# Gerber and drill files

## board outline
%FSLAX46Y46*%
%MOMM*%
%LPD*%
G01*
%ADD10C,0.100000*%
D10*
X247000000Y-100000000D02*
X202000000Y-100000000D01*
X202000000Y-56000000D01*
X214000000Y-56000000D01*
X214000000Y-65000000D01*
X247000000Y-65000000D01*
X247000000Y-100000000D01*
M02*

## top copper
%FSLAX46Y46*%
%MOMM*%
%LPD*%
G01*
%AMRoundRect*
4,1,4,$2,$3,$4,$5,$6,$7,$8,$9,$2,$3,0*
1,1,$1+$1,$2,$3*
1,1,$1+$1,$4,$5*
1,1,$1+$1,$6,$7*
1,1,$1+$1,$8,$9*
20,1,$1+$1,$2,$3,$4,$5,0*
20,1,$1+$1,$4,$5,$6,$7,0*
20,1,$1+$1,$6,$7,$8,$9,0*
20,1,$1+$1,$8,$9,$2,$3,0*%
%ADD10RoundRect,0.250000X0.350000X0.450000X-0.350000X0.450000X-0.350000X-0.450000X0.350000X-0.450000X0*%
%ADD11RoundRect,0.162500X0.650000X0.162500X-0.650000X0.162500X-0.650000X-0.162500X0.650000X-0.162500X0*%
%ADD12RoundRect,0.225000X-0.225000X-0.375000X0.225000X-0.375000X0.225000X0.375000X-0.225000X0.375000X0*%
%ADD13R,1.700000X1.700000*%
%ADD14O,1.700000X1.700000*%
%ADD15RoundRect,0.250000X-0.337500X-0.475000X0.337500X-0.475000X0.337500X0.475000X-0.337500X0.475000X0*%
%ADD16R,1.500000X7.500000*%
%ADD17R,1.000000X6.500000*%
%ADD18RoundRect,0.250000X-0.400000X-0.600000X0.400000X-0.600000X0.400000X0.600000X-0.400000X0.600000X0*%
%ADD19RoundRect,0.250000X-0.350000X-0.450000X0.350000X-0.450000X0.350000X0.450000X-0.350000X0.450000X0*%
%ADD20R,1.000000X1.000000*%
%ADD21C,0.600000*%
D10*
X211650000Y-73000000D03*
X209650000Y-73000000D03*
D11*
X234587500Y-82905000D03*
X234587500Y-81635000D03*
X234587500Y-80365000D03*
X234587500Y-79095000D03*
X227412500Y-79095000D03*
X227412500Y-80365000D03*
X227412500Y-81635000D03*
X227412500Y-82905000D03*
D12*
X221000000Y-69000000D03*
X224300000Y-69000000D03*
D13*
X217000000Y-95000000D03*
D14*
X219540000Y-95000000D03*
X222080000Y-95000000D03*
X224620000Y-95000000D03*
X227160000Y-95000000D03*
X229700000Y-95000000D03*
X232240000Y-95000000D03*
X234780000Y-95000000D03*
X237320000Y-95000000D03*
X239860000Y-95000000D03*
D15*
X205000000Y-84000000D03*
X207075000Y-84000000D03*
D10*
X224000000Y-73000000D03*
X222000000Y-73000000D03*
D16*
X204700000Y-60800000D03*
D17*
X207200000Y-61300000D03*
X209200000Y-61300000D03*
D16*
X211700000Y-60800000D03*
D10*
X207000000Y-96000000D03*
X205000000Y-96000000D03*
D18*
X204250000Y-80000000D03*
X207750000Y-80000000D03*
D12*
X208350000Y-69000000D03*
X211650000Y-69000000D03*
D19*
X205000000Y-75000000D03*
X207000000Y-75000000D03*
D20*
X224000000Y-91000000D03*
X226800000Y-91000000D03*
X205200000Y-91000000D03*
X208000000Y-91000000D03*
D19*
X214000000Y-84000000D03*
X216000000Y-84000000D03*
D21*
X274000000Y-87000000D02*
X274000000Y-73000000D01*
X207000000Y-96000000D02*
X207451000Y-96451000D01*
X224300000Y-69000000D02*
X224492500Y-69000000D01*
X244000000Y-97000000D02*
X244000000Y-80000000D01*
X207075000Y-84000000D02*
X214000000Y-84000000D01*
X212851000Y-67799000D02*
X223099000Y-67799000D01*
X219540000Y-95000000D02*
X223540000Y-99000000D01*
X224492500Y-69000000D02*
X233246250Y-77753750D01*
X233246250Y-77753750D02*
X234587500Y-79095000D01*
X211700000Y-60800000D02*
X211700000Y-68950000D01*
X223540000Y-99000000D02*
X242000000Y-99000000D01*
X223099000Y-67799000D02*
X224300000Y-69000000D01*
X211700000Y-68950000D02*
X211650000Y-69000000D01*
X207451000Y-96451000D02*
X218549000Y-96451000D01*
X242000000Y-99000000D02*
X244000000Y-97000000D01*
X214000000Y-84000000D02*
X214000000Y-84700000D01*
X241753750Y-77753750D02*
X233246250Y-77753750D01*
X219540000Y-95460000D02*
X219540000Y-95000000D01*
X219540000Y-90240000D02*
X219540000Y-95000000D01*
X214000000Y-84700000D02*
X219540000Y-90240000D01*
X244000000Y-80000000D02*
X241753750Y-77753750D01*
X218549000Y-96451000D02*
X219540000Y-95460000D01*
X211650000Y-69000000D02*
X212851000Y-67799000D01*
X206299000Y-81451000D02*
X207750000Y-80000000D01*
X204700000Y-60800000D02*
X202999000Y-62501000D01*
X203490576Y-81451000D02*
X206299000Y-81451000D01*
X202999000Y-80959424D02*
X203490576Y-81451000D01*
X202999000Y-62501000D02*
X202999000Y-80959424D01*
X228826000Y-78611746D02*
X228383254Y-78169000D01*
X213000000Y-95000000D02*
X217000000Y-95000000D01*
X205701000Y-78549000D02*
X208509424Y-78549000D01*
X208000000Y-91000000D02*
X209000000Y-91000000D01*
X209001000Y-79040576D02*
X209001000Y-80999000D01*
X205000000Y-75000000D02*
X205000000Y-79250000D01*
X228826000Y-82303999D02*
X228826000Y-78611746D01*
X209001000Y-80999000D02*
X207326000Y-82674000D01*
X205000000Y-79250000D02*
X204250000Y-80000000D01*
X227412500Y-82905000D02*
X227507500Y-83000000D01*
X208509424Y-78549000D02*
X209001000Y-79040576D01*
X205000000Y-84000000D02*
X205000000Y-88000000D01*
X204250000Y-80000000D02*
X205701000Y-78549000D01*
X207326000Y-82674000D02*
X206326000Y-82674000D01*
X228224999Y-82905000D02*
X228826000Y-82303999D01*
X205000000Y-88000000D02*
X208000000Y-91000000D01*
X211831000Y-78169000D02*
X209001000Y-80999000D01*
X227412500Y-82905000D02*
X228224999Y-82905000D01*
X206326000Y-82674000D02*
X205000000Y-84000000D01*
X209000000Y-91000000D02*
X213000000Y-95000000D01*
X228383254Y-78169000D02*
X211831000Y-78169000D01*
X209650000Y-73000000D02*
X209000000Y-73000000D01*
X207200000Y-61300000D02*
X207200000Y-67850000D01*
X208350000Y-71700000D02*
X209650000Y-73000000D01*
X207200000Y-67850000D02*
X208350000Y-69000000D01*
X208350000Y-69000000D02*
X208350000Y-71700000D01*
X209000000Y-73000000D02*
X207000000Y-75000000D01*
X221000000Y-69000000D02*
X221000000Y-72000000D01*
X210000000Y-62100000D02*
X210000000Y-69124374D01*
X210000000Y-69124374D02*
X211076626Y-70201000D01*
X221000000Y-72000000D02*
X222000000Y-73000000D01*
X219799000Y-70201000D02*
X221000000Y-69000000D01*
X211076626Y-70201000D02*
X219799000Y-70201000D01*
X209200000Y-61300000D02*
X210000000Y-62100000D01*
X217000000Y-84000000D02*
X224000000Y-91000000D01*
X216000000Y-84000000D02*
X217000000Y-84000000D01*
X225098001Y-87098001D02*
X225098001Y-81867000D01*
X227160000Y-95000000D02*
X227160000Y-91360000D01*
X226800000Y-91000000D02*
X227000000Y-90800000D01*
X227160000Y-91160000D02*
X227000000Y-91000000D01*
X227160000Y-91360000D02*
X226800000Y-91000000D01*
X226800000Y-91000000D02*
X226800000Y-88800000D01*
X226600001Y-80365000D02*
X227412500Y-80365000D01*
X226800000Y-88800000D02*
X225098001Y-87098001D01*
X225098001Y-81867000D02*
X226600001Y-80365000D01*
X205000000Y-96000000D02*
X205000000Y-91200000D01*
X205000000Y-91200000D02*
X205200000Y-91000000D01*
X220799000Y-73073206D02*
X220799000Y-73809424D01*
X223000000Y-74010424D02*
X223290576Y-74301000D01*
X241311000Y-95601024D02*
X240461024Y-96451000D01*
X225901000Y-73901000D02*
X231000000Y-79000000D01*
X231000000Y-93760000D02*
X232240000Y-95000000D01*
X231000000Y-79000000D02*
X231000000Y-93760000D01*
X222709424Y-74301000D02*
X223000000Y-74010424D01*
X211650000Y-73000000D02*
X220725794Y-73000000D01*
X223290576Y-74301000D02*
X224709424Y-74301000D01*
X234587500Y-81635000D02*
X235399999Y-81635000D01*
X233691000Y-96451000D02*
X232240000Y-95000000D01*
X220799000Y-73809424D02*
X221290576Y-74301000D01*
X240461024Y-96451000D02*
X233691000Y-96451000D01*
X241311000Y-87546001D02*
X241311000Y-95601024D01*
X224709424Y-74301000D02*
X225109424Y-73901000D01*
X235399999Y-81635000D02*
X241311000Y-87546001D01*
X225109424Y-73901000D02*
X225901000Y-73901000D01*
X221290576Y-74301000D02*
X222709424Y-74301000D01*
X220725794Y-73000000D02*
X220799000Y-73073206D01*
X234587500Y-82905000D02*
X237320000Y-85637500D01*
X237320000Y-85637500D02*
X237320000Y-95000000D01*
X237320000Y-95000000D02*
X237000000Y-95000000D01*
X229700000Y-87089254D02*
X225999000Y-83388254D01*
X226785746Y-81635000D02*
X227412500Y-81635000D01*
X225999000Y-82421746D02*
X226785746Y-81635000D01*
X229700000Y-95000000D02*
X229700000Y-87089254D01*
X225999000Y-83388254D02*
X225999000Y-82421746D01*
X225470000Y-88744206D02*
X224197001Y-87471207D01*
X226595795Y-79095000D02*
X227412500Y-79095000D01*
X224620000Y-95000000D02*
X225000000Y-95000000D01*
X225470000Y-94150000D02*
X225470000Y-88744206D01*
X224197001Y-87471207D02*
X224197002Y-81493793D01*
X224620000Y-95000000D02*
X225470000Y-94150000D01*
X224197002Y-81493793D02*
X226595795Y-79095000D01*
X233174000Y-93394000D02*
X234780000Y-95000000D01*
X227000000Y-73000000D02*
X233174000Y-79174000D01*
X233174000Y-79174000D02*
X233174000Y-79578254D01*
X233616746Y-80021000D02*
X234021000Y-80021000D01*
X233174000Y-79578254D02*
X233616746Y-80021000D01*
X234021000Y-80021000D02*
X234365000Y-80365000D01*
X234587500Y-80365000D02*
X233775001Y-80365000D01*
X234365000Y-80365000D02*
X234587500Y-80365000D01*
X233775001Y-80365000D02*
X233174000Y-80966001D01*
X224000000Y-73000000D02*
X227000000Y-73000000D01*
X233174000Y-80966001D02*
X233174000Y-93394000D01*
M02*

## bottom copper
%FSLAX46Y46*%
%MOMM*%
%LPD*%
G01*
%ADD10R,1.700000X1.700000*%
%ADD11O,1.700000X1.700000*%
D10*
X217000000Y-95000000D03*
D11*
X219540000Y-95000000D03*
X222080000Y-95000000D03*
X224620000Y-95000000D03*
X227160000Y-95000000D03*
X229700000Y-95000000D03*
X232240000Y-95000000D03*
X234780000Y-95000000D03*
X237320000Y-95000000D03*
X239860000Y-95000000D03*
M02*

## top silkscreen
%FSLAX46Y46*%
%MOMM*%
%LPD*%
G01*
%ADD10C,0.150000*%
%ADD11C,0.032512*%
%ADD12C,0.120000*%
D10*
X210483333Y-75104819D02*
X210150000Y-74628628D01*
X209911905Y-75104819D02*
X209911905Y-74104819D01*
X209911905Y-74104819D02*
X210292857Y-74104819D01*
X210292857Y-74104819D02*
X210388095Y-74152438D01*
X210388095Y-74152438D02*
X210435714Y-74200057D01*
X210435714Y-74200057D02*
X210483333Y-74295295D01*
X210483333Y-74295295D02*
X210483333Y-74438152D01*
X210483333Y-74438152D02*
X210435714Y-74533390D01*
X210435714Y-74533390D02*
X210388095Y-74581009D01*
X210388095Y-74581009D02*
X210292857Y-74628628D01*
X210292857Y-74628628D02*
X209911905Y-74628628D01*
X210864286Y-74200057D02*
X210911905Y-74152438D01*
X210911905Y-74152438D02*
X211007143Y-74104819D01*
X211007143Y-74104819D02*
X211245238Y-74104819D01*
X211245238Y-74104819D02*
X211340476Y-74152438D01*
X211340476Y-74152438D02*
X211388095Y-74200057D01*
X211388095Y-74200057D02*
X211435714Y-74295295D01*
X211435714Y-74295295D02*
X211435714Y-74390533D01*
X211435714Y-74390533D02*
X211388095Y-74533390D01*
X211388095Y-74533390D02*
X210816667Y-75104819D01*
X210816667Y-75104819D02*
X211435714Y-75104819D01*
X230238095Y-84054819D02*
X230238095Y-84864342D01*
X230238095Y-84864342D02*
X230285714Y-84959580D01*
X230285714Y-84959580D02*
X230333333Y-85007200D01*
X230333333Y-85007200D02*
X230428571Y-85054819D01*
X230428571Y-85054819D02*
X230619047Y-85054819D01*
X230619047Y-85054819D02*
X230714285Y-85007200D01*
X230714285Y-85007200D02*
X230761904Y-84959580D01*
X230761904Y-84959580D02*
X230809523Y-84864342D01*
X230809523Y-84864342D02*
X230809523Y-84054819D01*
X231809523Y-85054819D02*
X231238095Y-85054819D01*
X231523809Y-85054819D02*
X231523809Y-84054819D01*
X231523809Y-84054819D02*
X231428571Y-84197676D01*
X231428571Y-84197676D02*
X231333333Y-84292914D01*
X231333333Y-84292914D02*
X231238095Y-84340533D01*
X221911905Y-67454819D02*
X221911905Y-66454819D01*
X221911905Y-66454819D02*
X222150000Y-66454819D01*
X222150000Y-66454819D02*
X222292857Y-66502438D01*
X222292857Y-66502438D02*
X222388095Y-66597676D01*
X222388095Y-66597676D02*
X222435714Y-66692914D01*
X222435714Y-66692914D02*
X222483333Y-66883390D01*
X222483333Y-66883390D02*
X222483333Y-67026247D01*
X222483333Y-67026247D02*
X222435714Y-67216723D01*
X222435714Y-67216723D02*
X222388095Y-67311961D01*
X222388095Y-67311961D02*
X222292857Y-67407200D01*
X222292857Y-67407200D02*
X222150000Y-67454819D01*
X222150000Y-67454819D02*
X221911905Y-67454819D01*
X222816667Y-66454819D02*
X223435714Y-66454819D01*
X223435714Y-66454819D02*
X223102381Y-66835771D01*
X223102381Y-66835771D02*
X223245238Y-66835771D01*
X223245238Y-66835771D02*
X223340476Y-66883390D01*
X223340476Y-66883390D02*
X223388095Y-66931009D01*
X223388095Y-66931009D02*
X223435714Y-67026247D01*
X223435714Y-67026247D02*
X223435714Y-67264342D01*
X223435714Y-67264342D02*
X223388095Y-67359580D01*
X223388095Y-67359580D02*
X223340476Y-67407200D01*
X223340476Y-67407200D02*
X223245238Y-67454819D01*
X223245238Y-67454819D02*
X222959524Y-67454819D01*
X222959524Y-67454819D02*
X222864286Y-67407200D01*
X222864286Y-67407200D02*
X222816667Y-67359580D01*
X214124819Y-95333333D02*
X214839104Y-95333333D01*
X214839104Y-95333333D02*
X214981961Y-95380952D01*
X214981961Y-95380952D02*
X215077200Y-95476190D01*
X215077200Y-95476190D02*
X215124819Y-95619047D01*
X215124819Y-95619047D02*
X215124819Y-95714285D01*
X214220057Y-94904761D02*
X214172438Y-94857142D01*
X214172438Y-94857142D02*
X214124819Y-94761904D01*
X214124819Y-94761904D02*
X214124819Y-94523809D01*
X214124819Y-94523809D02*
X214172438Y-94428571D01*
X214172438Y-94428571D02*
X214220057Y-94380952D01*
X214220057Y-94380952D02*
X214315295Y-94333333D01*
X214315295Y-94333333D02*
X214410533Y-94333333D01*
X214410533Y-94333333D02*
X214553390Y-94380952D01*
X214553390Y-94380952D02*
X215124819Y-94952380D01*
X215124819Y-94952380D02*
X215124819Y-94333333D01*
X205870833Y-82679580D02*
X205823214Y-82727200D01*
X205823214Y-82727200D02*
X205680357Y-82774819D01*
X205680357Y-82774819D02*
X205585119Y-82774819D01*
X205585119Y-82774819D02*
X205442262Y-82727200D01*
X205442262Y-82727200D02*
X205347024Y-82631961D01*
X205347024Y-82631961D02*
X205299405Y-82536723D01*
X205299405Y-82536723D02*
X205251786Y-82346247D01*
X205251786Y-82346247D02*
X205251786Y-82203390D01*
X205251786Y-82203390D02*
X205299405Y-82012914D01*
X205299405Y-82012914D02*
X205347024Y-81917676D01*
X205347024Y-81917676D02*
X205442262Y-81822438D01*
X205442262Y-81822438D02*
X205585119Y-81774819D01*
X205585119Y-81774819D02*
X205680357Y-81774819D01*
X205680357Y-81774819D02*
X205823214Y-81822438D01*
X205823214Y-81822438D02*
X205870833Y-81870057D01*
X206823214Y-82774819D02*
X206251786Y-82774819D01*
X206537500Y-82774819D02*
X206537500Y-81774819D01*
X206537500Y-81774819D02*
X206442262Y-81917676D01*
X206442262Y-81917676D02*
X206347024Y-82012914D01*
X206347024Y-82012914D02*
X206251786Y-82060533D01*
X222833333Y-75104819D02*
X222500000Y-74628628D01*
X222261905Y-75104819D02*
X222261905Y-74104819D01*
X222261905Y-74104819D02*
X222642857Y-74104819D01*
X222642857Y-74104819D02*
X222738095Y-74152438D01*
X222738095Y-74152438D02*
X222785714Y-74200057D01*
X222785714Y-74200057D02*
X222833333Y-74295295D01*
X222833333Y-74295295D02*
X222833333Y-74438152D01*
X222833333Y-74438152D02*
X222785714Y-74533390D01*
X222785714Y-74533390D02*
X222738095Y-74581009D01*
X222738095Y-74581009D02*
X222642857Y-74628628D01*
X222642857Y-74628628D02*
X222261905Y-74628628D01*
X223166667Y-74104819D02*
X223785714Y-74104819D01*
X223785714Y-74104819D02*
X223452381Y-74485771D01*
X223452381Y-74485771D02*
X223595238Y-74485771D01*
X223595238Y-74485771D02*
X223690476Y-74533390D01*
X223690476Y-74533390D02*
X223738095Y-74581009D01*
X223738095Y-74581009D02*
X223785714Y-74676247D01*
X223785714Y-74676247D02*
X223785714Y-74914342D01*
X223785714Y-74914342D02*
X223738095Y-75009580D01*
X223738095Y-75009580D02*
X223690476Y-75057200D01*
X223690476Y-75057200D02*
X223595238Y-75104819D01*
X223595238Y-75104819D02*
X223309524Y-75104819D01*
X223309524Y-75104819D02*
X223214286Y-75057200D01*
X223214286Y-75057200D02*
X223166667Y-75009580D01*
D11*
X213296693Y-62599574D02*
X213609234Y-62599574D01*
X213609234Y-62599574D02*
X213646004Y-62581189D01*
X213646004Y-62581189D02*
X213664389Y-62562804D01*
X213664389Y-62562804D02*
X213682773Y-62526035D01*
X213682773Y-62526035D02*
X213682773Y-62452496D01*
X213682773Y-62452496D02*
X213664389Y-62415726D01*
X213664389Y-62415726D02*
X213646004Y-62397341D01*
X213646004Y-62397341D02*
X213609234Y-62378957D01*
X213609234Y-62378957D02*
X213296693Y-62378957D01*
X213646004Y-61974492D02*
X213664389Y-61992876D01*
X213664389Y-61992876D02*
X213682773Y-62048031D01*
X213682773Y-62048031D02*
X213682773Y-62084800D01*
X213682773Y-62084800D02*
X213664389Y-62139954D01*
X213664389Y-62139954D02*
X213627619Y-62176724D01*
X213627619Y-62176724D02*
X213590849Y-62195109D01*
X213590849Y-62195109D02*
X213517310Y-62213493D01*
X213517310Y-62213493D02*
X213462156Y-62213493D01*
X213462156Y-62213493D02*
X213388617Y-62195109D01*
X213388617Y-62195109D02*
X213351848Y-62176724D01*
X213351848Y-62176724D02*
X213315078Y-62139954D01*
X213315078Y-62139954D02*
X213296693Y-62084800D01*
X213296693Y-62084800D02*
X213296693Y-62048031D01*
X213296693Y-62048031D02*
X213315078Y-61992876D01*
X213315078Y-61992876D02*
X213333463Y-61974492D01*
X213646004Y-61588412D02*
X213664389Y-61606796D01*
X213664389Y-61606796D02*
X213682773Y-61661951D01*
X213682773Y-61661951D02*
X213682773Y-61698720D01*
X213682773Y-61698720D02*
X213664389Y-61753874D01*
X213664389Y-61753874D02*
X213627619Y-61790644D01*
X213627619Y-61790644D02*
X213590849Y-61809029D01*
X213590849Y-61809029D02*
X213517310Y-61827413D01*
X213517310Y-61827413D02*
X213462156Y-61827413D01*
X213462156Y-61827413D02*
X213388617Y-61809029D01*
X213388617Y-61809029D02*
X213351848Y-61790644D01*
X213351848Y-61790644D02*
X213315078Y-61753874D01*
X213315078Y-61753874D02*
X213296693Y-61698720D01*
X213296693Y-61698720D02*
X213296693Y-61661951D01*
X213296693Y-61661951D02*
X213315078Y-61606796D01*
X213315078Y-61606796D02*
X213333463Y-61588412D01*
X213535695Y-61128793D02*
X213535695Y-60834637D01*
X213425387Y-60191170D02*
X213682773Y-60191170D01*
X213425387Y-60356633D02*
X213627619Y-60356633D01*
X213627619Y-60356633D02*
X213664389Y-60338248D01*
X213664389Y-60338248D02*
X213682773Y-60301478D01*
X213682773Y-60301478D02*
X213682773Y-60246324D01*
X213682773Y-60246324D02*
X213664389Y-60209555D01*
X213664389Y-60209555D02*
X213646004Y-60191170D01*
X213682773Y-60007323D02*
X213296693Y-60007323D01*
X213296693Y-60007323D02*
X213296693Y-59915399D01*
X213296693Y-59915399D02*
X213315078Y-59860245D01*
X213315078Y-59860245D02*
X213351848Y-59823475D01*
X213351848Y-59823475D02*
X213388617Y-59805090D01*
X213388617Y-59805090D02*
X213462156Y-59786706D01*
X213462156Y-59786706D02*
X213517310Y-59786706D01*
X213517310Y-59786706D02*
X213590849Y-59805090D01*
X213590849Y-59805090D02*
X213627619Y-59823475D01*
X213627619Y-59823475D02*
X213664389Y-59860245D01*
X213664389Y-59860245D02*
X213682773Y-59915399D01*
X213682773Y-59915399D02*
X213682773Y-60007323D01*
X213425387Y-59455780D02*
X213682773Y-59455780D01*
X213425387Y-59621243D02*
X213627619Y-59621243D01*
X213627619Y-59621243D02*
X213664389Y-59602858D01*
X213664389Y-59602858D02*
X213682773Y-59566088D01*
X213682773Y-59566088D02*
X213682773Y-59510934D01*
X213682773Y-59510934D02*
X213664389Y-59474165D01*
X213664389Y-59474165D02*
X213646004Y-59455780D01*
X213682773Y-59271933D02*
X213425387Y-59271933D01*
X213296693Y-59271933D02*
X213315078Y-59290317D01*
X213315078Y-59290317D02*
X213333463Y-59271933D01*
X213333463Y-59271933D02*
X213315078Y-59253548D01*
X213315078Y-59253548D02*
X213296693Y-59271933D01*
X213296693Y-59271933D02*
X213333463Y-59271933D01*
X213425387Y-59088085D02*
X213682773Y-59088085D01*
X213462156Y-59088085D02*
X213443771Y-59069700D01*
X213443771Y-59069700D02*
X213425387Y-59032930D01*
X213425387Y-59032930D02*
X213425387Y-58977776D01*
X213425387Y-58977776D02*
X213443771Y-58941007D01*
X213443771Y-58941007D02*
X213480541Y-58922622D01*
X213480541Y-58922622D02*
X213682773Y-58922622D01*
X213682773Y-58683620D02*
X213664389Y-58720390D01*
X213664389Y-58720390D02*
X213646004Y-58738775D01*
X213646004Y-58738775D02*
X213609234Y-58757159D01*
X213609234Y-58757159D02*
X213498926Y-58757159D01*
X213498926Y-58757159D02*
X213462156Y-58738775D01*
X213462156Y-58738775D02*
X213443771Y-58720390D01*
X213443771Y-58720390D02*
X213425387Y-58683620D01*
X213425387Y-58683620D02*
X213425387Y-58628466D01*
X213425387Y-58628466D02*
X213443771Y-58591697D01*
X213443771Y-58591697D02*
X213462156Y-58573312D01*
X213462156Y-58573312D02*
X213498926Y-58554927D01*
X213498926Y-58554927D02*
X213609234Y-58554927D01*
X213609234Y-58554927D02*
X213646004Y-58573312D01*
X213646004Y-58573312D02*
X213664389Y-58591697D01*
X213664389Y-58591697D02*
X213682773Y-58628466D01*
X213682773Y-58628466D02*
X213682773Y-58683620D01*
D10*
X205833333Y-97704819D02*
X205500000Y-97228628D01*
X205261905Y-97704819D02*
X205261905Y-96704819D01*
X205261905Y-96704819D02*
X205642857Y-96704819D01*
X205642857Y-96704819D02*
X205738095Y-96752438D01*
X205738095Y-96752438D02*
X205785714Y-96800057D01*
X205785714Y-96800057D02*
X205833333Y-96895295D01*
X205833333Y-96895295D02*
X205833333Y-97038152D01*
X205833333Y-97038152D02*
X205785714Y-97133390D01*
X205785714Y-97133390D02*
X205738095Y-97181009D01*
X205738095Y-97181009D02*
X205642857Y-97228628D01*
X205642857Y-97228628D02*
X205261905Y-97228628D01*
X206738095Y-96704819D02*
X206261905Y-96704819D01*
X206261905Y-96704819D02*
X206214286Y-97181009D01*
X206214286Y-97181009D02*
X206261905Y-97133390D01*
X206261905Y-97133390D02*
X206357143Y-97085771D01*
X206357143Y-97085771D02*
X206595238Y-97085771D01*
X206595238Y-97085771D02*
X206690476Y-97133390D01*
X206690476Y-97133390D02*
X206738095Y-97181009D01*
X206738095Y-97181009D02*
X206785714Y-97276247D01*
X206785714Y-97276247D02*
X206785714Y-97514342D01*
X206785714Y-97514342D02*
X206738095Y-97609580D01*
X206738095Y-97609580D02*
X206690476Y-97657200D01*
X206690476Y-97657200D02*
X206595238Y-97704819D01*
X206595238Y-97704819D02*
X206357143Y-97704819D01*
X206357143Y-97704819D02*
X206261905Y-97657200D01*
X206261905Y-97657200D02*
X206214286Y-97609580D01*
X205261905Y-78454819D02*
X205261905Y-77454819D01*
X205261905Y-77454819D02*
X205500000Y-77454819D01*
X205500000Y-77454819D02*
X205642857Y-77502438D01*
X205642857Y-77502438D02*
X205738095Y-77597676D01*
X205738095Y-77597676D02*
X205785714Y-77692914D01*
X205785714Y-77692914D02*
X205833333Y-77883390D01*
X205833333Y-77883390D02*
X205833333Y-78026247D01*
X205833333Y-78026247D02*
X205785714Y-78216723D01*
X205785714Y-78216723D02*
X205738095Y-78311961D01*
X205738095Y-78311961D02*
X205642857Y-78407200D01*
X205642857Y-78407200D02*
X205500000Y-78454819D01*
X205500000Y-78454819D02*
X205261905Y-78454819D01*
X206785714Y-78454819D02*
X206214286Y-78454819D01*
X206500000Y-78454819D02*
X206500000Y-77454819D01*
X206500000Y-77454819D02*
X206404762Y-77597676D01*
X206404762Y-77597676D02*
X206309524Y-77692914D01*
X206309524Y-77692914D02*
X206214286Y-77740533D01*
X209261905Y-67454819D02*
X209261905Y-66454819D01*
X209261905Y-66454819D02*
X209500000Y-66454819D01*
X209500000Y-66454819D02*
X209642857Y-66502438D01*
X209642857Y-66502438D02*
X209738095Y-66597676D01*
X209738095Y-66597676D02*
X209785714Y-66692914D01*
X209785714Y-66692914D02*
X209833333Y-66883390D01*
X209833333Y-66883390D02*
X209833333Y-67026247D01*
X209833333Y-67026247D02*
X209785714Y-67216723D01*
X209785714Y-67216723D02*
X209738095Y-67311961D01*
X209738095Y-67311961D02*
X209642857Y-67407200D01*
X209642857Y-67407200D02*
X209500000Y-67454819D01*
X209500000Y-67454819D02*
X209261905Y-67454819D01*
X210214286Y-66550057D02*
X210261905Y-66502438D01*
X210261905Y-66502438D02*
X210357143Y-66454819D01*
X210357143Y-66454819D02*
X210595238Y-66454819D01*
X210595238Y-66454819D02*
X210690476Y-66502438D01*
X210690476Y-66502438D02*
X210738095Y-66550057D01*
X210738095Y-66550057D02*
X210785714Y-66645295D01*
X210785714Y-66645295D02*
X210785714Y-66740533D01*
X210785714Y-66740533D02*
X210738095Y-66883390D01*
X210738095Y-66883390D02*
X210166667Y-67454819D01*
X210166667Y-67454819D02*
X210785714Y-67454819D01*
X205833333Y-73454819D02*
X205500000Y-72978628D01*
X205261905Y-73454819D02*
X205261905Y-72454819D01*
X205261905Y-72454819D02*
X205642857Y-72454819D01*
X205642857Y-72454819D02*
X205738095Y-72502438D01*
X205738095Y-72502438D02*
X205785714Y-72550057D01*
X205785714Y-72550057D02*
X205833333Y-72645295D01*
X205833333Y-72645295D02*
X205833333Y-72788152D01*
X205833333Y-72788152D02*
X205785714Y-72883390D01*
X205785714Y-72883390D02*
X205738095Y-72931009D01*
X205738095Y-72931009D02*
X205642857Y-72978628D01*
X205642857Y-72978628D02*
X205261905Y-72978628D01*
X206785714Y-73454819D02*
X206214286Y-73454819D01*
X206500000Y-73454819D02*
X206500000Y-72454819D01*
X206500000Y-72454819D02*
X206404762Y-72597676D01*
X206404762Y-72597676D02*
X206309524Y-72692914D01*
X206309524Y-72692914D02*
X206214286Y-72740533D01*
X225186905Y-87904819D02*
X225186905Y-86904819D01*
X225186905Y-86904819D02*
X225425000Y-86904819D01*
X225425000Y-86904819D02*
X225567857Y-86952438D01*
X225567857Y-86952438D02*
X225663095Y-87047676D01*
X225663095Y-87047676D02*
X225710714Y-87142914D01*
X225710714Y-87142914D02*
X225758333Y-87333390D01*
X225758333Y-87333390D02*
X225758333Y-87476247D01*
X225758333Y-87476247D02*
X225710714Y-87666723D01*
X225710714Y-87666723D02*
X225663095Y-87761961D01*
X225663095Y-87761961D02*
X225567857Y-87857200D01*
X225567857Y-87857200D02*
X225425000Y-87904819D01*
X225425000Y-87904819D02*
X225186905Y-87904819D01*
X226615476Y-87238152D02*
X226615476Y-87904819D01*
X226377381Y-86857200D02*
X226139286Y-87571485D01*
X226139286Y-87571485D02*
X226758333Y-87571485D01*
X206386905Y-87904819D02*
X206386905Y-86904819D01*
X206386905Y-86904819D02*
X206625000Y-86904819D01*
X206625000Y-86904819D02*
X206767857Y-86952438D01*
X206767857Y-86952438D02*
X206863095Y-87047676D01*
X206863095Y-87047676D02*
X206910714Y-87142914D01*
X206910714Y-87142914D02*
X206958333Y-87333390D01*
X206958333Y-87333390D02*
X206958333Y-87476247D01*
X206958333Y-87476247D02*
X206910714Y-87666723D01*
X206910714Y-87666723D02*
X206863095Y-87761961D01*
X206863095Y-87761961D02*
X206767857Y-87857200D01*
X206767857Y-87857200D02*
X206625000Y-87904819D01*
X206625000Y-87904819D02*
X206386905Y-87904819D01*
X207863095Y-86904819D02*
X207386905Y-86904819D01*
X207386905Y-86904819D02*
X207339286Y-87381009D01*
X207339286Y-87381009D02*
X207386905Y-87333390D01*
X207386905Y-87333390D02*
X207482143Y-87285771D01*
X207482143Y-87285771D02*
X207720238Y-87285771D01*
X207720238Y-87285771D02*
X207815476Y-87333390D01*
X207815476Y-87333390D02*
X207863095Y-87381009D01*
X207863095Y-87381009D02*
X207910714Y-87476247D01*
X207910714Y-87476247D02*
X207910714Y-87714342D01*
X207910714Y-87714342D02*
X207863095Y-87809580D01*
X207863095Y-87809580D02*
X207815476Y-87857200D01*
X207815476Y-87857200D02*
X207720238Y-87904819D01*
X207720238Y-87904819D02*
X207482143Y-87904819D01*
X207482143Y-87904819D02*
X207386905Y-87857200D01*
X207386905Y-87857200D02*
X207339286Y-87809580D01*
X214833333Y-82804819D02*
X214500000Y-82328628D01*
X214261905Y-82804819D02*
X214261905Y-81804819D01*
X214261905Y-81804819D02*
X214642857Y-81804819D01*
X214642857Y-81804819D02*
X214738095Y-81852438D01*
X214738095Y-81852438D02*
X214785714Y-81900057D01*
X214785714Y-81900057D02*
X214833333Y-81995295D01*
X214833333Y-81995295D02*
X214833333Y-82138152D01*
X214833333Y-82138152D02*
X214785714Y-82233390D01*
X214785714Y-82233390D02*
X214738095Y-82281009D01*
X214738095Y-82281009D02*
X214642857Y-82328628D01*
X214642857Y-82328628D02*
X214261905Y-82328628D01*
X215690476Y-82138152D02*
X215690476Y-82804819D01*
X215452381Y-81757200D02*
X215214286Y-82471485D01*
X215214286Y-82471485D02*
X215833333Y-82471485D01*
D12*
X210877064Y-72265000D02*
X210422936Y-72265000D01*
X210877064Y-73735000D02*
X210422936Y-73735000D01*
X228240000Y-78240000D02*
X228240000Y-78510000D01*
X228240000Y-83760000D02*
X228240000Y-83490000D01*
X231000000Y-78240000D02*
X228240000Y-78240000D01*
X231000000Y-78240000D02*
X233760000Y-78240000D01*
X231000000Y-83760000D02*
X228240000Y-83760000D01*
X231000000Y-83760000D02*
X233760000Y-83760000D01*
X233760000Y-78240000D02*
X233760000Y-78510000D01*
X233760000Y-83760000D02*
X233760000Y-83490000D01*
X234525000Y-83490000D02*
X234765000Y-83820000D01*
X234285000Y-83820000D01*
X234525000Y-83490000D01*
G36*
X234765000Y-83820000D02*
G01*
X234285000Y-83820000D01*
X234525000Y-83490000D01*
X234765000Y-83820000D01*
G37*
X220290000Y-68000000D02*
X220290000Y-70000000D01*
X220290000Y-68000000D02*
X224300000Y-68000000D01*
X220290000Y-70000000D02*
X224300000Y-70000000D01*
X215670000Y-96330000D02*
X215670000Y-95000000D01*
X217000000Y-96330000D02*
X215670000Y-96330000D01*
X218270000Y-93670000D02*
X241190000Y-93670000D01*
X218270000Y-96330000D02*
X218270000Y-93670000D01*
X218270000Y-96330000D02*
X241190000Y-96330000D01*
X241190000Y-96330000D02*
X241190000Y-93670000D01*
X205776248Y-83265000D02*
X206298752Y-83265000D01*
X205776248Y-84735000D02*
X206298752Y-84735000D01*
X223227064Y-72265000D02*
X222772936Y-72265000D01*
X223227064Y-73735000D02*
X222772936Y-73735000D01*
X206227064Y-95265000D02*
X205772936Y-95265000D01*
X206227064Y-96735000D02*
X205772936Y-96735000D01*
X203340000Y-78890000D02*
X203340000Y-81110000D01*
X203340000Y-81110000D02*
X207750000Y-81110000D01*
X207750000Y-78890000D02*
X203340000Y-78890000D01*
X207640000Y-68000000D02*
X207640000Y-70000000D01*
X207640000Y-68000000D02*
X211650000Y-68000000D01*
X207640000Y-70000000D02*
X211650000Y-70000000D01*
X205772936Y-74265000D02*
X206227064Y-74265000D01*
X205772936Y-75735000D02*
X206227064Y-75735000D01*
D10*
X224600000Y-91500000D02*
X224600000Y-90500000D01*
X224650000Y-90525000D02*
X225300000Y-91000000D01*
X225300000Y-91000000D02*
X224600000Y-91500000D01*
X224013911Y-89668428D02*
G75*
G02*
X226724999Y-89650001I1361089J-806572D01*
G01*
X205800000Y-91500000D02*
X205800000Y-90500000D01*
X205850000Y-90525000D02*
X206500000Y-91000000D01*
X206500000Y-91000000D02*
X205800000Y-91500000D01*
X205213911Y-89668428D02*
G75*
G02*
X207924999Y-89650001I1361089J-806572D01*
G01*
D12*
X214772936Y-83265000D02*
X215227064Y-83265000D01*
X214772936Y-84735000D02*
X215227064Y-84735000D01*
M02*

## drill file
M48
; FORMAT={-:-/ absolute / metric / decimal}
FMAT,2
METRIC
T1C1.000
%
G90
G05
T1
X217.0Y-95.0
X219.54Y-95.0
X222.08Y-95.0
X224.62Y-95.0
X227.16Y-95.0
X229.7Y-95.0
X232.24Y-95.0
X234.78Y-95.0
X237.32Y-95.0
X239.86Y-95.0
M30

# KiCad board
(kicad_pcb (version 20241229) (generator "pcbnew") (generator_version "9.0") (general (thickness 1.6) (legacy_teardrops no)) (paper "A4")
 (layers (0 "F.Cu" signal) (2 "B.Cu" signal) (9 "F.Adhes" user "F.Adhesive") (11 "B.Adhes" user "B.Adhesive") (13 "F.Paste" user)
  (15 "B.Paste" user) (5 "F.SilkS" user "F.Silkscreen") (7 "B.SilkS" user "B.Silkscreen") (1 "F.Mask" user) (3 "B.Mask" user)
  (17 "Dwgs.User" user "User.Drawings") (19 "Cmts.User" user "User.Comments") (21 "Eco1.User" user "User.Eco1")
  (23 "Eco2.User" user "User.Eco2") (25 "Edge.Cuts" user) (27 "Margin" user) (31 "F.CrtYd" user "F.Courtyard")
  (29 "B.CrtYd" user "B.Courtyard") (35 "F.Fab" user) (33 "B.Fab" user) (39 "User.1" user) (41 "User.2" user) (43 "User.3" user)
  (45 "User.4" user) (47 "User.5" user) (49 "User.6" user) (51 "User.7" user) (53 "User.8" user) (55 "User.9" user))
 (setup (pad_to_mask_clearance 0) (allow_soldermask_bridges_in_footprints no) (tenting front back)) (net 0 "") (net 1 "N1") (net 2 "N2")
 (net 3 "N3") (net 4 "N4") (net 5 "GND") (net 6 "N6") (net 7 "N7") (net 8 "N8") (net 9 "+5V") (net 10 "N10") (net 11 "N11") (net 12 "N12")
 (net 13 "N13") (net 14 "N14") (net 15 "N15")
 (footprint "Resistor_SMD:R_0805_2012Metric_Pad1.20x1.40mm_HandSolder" (layer "F.Cu") (at 210.65 73 180)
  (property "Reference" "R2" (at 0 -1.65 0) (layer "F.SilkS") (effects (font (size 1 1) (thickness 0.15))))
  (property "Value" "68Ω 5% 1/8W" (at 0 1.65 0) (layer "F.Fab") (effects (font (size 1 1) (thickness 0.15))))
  (fp_line (start -0.227064 0.735) (end 0.227064 0.735) (stroke (width 0.12) (type solid)) (layer "F.SilkS"))
  (fp_line (start -0.227064 -0.735) (end 0.227064 -0.735) (stroke (width 0.12) (type solid)) (layer "F.SilkS"))
  (pad "1" smd roundrect (at -1 0 180) (size 1.2 1.4) (layers "F.Cu" "F.Mask" "F.Paste") (roundrect_rratio 0.208333) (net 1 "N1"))
  (pad "2" smd roundrect (at 1 0 180) (size 1.2 1.4) (layers "F.Cu" "F.Mask" "F.Paste") (roundrect_rratio 0.208333) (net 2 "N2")))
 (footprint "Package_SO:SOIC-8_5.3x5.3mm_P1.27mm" (layer "F.Cu") (at 231 81 180)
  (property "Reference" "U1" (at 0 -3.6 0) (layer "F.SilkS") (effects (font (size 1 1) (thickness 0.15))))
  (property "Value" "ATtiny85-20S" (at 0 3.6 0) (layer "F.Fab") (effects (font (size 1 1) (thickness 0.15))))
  (fp_line (start 2.76 2.76) (end 2.76 2.49) (stroke (width 0.12) (type solid)) (layer "F.SilkS"))
  (fp_line (start 2.76 -2.76) (end 2.76 -2.49) (stroke (width 0.12) (type solid)) (layer "F.SilkS"))
  (fp_line (start 0 2.76) (end 2.76 2.76) (stroke (width 0.12) (type solid)) (layer "F.SilkS"))
  (fp_line (start 0 2.76) (end -2.76 2.76) (stroke (width 0.12) (type solid)) (layer "F.SilkS"))
  (fp_line (start 0 -2.76) (end 2.76 -2.76) (stroke (width 0.12) (type solid)) (layer "F.SilkS"))
  (fp_line (start 0 -2.76) (end -2.76 -2.76) (stroke (width 0.12) (type solid)) (layer "F.SilkS"))
  (fp_line (start -2.76 2.76) (end -2.76 2.49) (stroke (width 0.12) (type solid)) (layer "F.SilkS"))
  (fp_line (start -2.76 -2.76) (end -2.76 -2.49) (stroke (width 0.12) (type solid)) (layer "F.SilkS"))
  (fp_poly
   (pts (xy -3.525 -2.49) (xy -3.765 -2.82) (xy -3.285 -2.82) (xy -3.525 -2.49)) (stroke (width 0.12) (type solid)) (fill yes)
   (layer "F.SilkS"))
  (pad "1" smd roundrect (at -3.5875 -1.905 180) (size 1.625 0.65) (layers "F.Cu" "F.Mask" "F.Paste") (roundrect_rratio 0.25) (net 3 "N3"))
  (pad "2" smd roundrect (at -3.5875 -0.635 180) (size 1.625 0.65) (layers "F.Cu" "F.Mask" "F.Paste") (roundrect_rratio 0.25) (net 1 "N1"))
  (pad "3" smd roundrect (at -3.5875 0.635 180) (size 1.625 0.65) (layers "F.Cu" "F.Mask" "F.Paste") (roundrect_rratio 0.25) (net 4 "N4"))
  (pad "4" smd roundrect (at -3.5875 1.905 180) (size 1.625 0.65) (layers "F.Cu" "F.Mask" "F.Paste") (roundrect_rratio 0.25) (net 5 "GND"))
  (pad "5" smd roundrect (at 3.5875 1.905 180) (size 1.625 0.65) (layers "F.Cu" "F.Mask" "F.Paste") (roundrect_rratio 0.25) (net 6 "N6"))
  (pad "6" smd roundrect (at 3.5875 0.635 180) (size 1.625 0.65) (layers "F.Cu" "F.Mask" "F.Paste") (roundrect_rratio 0.25) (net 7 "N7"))
  (pad "7" smd roundrect (at 3.5875 -0.635 180) (size 1.625 0.65) (layers "F.Cu" "F.Mask" "F.Paste") (roundrect_rratio 0.25) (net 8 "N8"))
  (pad "8" smd roundrect (at 3.5875 -1.905 180) (size 1.625 0.65) (layers "F.Cu" "F.Mask" "F.Paste") (roundrect_rratio 0.25) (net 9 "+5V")))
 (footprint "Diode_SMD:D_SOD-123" (layer "F.Cu") (at 222.65 69)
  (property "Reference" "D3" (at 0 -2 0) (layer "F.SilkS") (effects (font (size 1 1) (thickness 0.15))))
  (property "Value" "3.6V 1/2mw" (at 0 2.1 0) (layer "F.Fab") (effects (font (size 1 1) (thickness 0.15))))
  (fp_line (start -2.36 -1) (end -2.36 1) (stroke (width 0.12) (type solid)) (layer "F.SilkS"))
  (fp_line (start -2.36 -1) (end 1.65 -1) (stroke (width 0.12) (type solid)) (layer "F.SilkS"))
  (fp_line (start -2.36 1) (end 1.65 1) (stroke (width 0.12) (type solid)) (layer "F.SilkS"))
  (pad "1" smd roundrect (at -1.65 0) (size 0.9 1.2) (layers "F.Cu" "F.Mask" "F.Paste") (roundrect_rratio 0.25) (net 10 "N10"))
  (pad "2" smd roundrect (at 1.65 0) (size 0.9 1.2) (layers "F.Cu" "F.Mask" "F.Paste") (roundrect_rratio 0.25) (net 5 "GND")))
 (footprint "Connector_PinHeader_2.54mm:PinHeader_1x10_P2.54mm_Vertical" (layer "F.Cu") (at 217 95 90)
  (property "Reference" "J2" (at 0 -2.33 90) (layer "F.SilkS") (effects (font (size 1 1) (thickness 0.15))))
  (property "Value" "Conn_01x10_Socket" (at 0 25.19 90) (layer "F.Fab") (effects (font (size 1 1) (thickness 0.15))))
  (fp_line (start -1.33 -1.33) (end 0 -1.33) (stroke (width 0.12) (type solid)) (layer "F.SilkS"))
  (fp_line (start -1.33 0) (end -1.33 -1.33) (stroke (width 0.12) (type solid)) (layer "F.SilkS"))
  (fp_line (start 1.33 1.27) (end 1.33 24.19) (stroke (width 0.12) (type solid)) (layer "F.SilkS"))
  (fp_line (start -1.33 1.27) (end 1.33 1.27) (stroke (width 0.12) (type solid)) (layer "F.SilkS"))
  (fp_line (start -1.33 1.27) (end -1.33 24.19) (stroke (width 0.12) (type solid)) (layer "F.SilkS"))
  (fp_line (start -1.33 24.19) (end 1.33 24.19) (stroke (width 0.12) (type solid)) (layer "F.SilkS"))
  (pad "1" thru_hole rect (at 0 0 90) (size 1.7 1.7) (drill 1) (layers "*.Cu" "*.Mask") (remove_unused_layers no) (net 9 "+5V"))
  (pad "2" thru_hole oval (at 0 2.54 90) (size 1.7 1.7) (drill 1) (layers "*.Cu" "*.Mask") (remove_unused_layers no) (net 5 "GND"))
  (pad "3" thru_hole oval (at 0 5.08 90) (size 1.7 1.7) (drill 1) (layers "*.Cu" "*.Mask") (remove_unused_layers no) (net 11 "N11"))
  (pad "4" thru_hole oval (at 0 7.62 90) (size 1.7 1.7) (drill 1) (layers "*.Cu" "*.Mask") (remove_unused_layers no) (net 6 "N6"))
  (pad "5" thru_hole oval (at 0 10.16 90) (size 1.7 1.7) (drill 1) (layers "*.Cu" "*.Mask") (remove_unused_layers no) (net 7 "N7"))
  (pad "6" thru_hole oval (at 0 12.7 90) (size 1.7 1.7) (drill 1) (layers "*.Cu" "*.Mask") (remove_unused_layers no) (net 8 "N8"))
  (pad "7" thru_hole oval (at 0 15.24 90) (size 1.7 1.7) (drill 1) (layers "*.Cu" "*.Mask") (remove_unused_layers no) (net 1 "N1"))
  (pad "8" thru_hole oval (at 0 17.78 90) (size 1.7 1.7) (drill 1) (layers "*.Cu" "*.Mask") (remove_unused_layers no) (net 4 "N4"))
  (pad "9" thru_hole oval (at 0 20.32 90) (size 1.7 1.7) (drill 1) (layers "*.Cu" "*.Mask") (remove_unused_layers no) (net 3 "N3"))
  (pad "10" thru_hole oval (at 0 22.86 90) (size 1.7 1.7) (drill 1) (layers "*.Cu" "*.Mask") (remove_unused_layers no) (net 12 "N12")))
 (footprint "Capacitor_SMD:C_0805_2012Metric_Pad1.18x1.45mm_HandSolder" (layer "F.Cu") (at 206.0375 84)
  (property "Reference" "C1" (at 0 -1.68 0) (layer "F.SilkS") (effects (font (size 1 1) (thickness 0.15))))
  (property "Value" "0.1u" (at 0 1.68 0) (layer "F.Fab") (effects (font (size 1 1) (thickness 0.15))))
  (fp_line (start -0.261252 -0.735) (end 0.261252 -0.735) (stroke (width 0.12) (type solid)) (layer "F.SilkS"))
  (fp_line (start -0.261252 0.735) (end 0.261252 0.735) (stroke (width 0.12) (type solid)) (layer "F.SilkS"))
  (pad "1" smd roundrect (at -1.0375 0) (size 1.175 1.45) (layers "F.Cu" "F.Mask" "F.Paste") (roundrect_rratio 0.212766) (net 9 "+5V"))
  (pad "2" smd roundrect (at 1.0375 0) (size 1.175 1.45) (layers "F.Cu" "F.Mask" "F.Paste") (roundrect_rratio 0.212766) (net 5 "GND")))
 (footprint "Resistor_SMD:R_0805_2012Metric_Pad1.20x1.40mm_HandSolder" (layer "F.Cu") (at 223 73 180)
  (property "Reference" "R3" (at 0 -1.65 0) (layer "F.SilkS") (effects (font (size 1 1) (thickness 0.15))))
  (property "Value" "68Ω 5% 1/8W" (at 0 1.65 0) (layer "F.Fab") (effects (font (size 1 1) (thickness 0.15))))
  (fp_line (start -0.227064 0.735) (end 0.227064 0.735) (stroke (width 0.12) (type solid)) (layer "F.SilkS"))
  (fp_line (start -0.227064 -0.735) (end 0.227064 -0.735) (stroke (width 0.12) (type solid)) (layer "F.SilkS"))
  (pad "1" smd roundrect (at -1 0 180) (size 1.2 1.4) (layers "F.Cu" "F.Mask" "F.Paste") (roundrect_rratio 0.208333) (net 4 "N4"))
  (pad "2" smd roundrect (at 1 0 180) (size 1.2 1.4) (layers "F.Cu" "F.Mask" "F.Paste") (roundrect_rratio 0.208333) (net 10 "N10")))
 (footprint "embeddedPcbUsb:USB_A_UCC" (layer "F.Cu") (at 208.2 61 -90)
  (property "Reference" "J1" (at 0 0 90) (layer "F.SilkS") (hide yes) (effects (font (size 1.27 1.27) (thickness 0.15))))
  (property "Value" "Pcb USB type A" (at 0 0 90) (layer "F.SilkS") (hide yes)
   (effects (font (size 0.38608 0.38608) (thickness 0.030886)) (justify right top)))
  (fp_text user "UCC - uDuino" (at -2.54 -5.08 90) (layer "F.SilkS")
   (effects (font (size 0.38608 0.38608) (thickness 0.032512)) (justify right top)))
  (pad "1" smd rect (at -0.2 3.5 270) (size 7.5 1.5) (layers "F.Cu" "F.Mask" "F.Paste") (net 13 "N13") (solder_mask_margin 0.1016))
  (pad "2" smd rect (at 0.3 1 270) (size 6.5 1) (layers "F.Cu" "F.Mask" "F.Paste") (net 2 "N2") (solder_mask_margin 0.1016))
  (pad "3" smd rect (at 0.3 -1 270) (size 6.5 1) (layers "F.Cu" "F.Mask" "F.Paste") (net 10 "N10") (solder_mask_margin 0.1016))
  (pad "4" smd rect (at -0.2 -3.5 270) (size 7.5 1.5) (layers "F.Cu" "F.Mask" "F.Paste") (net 5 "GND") (solder_mask_margin 0.1016)))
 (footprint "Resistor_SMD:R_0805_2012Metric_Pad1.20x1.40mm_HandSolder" (layer "F.Cu") (at 206 96 180)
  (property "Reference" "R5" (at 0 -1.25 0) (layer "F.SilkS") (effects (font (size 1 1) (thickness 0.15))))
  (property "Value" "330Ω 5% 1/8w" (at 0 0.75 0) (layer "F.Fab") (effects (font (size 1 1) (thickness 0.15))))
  (fp_line (start -0.227064 0.735) (end 0.227064 0.735) (stroke (width 0.12) (type solid)) (layer "F.SilkS"))
  (fp_line (start -0.227064 -0.735) (end 0.227064 -0.735) (stroke (width 0.12) (type solid)) (layer "F.SilkS"))
  (pad "1" smd roundrect (at -1 0 180) (size 1.2 1.4) (layers "F.Cu" "F.Mask" "F.Paste") (roundrect_rratio 0.208333) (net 5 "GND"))
  (pad "2" smd roundrect (at 1 0 180) (size 1.2 1.4) (layers "F.Cu" "F.Mask" "F.Paste") (roundrect_rratio 0.208333) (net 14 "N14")))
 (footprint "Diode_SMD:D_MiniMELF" (layer "F.Cu") (at 206 80)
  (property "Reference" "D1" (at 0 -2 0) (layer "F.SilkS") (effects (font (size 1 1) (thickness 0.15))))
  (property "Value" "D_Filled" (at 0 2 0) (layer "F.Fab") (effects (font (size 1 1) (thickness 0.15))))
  (fp_line (start -2.66 -1.11) (end -2.66 1.11) (stroke (width 0.12) (type solid)) (layer "F.SilkS"))
  (fp_line (start -2.66 1.11) (end 1.75 1.11) (stroke (width 0.12) (type solid)) (layer "F.SilkS"))
  (fp_line (start 1.75 -1.11) (end -2.66 -1.11) (stroke (width 0.12) (type solid)) (layer "F.SilkS"))
  (pad "1" smd roundrect (at -1.75 0) (size 1.3 1.7) (layers "F.Cu" "F.Mask" "F.Paste") (roundrect_rratio 0.1923076923) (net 9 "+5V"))
  (pad "2" smd roundrect (at 1.75 0) (size 1.3 1.7) (layers "F.Cu" "F.Mask" "F.Paste") (roundrect_rratio 0.1923076923) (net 13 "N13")))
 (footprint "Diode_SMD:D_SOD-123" (layer "F.Cu") (at 210 69)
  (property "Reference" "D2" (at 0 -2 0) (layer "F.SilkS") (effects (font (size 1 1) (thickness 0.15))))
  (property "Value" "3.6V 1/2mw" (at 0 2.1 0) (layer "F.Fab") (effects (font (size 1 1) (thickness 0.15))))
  (fp_line (start -2.36 -1) (end -2.36 1) (stroke (width 0.12) (type solid)) (layer "F.SilkS"))
  (fp_line (start -2.36 -1) (end 1.65 -1) (stroke (width 0.12) (type solid)) (layer "F.SilkS"))
  (fp_line (start -2.36 1) (end 1.65 1) (stroke (width 0.12) (type solid)) (layer "F.SilkS"))
  (pad "1" smd roundrect (at -1.65 0) (size 0.9 1.2) (layers "F.Cu" "F.Mask" "F.Paste") (roundrect_rratio 0.25) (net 2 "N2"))
  (pad "2" smd roundrect (at 1.65 0) (size 0.9 1.2) (layers "F.Cu" "F.Mask" "F.Paste") (roundrect_rratio 0.25) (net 5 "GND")))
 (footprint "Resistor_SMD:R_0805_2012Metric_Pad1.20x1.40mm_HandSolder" (layer "F.Cu") (at 206 75)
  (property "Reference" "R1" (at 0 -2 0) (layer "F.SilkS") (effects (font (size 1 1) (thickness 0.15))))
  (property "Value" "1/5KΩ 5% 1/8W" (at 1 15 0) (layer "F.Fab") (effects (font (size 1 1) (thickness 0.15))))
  (fp_line (start -0.227064 -0.735) (end 0.227064 -0.735) (stroke (width 0.12) (type solid)) (layer "F.SilkS"))
  (fp_line (start -0.227064 0.735) (end 0.227064 0.735) (stroke (width 0.12) (type solid)) (layer "F.SilkS"))
  (pad "1" smd roundrect (at -1 0) (size 1.2 1.4) (layers "F.Cu" "F.Mask" "F.Paste") (roundrect_rratio 0.208333) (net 9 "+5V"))
  (pad "2" smd roundrect (at 1 0) (size 1.2 1.4) (layers "F.Cu" "F.Mask" "F.Paste") (roundrect_rratio 0.208333) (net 2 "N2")))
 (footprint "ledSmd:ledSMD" (layer "F.Cu") (at 225.8 91)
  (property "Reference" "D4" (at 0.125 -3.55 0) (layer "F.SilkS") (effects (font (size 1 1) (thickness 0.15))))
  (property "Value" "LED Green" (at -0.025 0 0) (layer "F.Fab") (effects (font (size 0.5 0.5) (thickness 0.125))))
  (fp_line (start -1.2 0.5) (end -1.2 -0.5) (stroke (width 0.15) (type solid)) (layer "F.SilkS"))
  (fp_line (start -1.15 -0.475) (end -0.5 0) (stroke (width 0.15) (type solid)) (layer "F.SilkS"))
  (fp_line (start -0.5 0) (end -1.2 0.5) (stroke (width 0.15) (type solid)) (layer "F.SilkS"))
  (fp_arc (start -1.786089 -1.331572) (mid -0.435753 -2.107089) (end 0.924999 -1.349999) (stroke (width 0.15) (type solid))
   (layer "F.SilkS"))
  (pad "1" smd rect (at -1.8 0) (size 1 1) (layers "F.Cu" "F.Mask" "F.Paste") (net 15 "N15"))
  (pad "2" smd rect (at 1 0) (size 1 1) (layers "F.Cu" "F.Mask" "F.Paste") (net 7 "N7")))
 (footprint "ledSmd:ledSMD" (layer "F.Cu") (at 207 91)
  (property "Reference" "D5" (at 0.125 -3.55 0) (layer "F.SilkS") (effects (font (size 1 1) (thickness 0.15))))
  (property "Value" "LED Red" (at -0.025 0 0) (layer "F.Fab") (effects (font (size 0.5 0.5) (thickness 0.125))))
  (fp_line (start -1.2 0.5) (end -1.2 -0.5) (stroke (width 0.15) (type solid)) (layer "F.SilkS"))
  (fp_line (start -1.15 -0.475) (end -0.5 0) (stroke (width 0.15) (type solid)) (layer "F.SilkS"))
  (fp_line (start -0.5 0) (end -1.2 0.5) (stroke (width 0.15) (type solid)) (layer "F.SilkS"))
  (fp_arc (start -1.786089 -1.331572) (mid -0.435753 -2.107089) (end 0.924999 -1.349999) (stroke (width 0.15) (type solid))
   (layer "F.SilkS"))
  (pad "1" smd rect (at -1.8 0) (size 1 1) (layers "F.Cu" "F.Mask" "F.Paste") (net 14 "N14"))
  (pad "2" smd rect (at 1 0) (size 1 1) (layers "F.Cu" "F.Mask" "F.Paste") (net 9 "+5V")))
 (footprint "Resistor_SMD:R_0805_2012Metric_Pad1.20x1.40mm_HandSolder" (layer "F.Cu") (at 215 84)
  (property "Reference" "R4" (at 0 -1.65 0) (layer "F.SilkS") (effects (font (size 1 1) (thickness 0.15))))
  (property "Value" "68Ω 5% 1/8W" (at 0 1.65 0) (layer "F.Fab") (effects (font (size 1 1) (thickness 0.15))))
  (fp_line (start -0.227064 -0.735) (end 0.227064 -0.735) (stroke (width 0.12) (type solid)) (layer "F.SilkS"))
  (fp_line (start -0.227064 0.735) (end 0.227064 0.735) (stroke (width 0.12) (type solid)) (layer "F.SilkS"))
  (pad "1" smd roundrect (at -1 0) (size 1.2 1.4) (layers "F.Cu" "F.Mask" "F.Paste") (roundrect_rratio 0.208333) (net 5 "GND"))
  (pad "2" smd roundrect (at 1 0) (size 1.2 1.4) (layers "F.Cu" "F.Mask" "F.Paste") (roundrect_rratio 0.208333) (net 15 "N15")))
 (gr_poly
  (pts (xy 247 100) (xy 202 100) (xy 202 56) (xy 214 56) (xy 214 65) (xy 247 65)) (stroke (width 0.1) (type solid)) (fill no)
  (layer "Edge.Cuts"))
 (segment (start 274 87) (end 274 73) (width 0.6) (layer "F.Cu") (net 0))
 (segment (start 207 96) (end 207.451 96.451) (width 0.6) (layer "F.Cu") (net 5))
 (segment (start 224.3 69) (end 224.4925 69) (width 0.6) (layer "F.Cu") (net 5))
 (segment (start 244 97) (end 244 80) (width 0.6) (layer "F.Cu") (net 5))
 (segment (start 207.075 84) (end 214 84) (width 0.6) (layer "F.Cu") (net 5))
 (segment (start 212.851 67.799) (end 223.099 67.799) (width 0.6) (layer "F.Cu") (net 5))
 (segment (start 219.54 95) (end 223.54 99) (width 0.6) (layer "F.Cu") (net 5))
 (segment (start 224.4925 69) (end 233.24625 77.75375) (width 0.6) (layer "F.Cu") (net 5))
 (segment (start 233.24625 77.75375) (end 234.5875 79.095) (width 0.6) (layer "F.Cu") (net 5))
 (segment (start 211.7 60.8) (end 211.7 68.95) (width 0.6) (layer "F.Cu") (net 5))
 (segment (start 223.54 99) (end 242 99) (width 0.6) (layer "F.Cu") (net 5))
 (segment (start 223.099 67.799) (end 224.3 69) (width 0.6) (layer "F.Cu") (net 5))
 (segment (start 211.7 68.95) (end 211.65 69) (width 0.6) (layer "F.Cu") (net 5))
 (segment (start 207.451 96.451) (end 218.549 96.451) (width 0.6) (layer "F.Cu") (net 5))
 (segment (start 242 99) (end 244 97) (width 0.6) (layer "F.Cu") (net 5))
 (segment (start 214 84) (end 214 84.7) (width 0.6) (layer "F.Cu") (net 5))
 (segment (start 241.75375 77.75375) (end 233.24625 77.75375) (width 0.6) (layer "F.Cu") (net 5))
 (segment (start 219.54 95.46) (end 219.54 95) (width 0.6) (layer "F.Cu") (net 5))
 (segment (start 219.54 90.24) (end 219.54 95) (width 0.6) (layer "F.Cu") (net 5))
 (segment (start 214 84.7) (end 219.54 90.24) (width 0.6) (layer "F.Cu") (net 5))
 (segment (start 244 80) (end 241.75375 77.75375) (width 0.6) (layer "F.Cu") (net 5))
 (segment (start 218.549 96.451) (end 219.54 95.46) (width 0.6) (layer "F.Cu") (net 5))
 (segment (start 211.65 69) (end 212.851 67.799) (width 0.6) (layer "F.Cu") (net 5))
 (segment (start 206.299 81.451) (end 207.75 80) (width 0.6) (layer "F.Cu") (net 13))
 (segment (start 204.7 60.8) (end 202.999 62.501) (width 0.6) (layer "F.Cu") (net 13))
 (segment (start 203.490576 81.451) (end 206.299 81.451) (width 0.6) (layer "F.Cu") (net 13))
 (segment (start 202.999 80.959424) (end 203.490576 81.451) (width 0.6) (layer "F.Cu") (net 13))
 (segment (start 202.999 62.501) (end 202.999 80.959424) (width 0.6) (layer "F.Cu") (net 13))
 (segment (start 228.826 78.611746) (end 228.383254 78.169) (width 0.6) (layer "F.Cu") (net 9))
 (segment (start 213 95) (end 217 95) (width 0.6) (layer "F.Cu") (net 9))
 (segment (start 205.701 78.549) (end 208.509424 78.549) (width 0.6) (layer "F.Cu") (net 9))
 (segment (start 208 91) (end 209 91) (width 0.6) (layer "F.Cu") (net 9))
 (segment (start 209.001 79.040576) (end 209.001 80.999) (width 0.6) (layer "F.Cu") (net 9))
 (segment (start 205 75) (end 205 79.25) (width 0.6) (layer "F.Cu") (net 9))
 (segment (start 228.826 82.303999) (end 228.826 78.611746) (width 0.6) (layer "F.Cu") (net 9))
 (segment (start 209.001 80.999) (end 207.326 82.674) (width 0.6) (layer "F.Cu") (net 9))
 (segment (start 205 79.25) (end 204.25 80) (width 0.6) (layer "F.Cu") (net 9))
 (segment (start 227.4125 82.905) (end 227.5075 83) (width 0.6) (layer "F.Cu") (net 9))
 (segment (start 208.509424 78.549) (end 209.001 79.040576) (width 0.6) (layer "F.Cu") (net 9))
 (segment (start 205 84) (end 205 88) (width 0.6) (layer "F.Cu") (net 9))
 (segment (start 204.25 80) (end 205.701 78.549) (width 0.6) (layer "F.Cu") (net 9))
 (segment (start 207.326 82.674) (end 206.326 82.674) (width 0.6) (layer "F.Cu") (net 9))
 (segment (start 228.224999 82.905) (end 228.826 82.303999) (width 0.6) (layer "F.Cu") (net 9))
 (segment (start 205 88) (end 208 91) (width 0.6) (layer "F.Cu") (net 9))
 (segment (start 211.831 78.169) (end 209.001 80.999) (width 0.6) (layer "F.Cu") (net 9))
 (segment (start 227.4125 82.905) (end 228.224999 82.905) (width 0.6) (layer "F.Cu") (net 9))
 (segment (start 206.326 82.674) (end 205 84) (width 0.6) (layer "F.Cu") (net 9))
 (segment (start 209 91) (end 213 95) (width 0.6) (layer "F.Cu") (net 9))
 (segment (start 228.383254 78.169) (end 211.831 78.169) (width 0.6) (layer "F.Cu") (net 9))
 (segment (start 209.65 73) (end 209 73) (width 0.6) (layer "F.Cu") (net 2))
 (segment (start 207.2 61.3) (end 207.2 67.85) (width 0.6) (layer "F.Cu") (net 2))
 (segment (start 208.35 71.7) (end 209.65 73) (width 0.6) (layer "F.Cu") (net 2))
 (segment (start 207.2 67.85) (end 208.35 69) (width 0.6) (layer "F.Cu") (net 2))
 (segment (start 208.35 69) (end 208.35 71.7) (width 0.6) (layer "F.Cu") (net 2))
 (segment (start 209 73) (end 207 75) (width 0.6) (layer "F.Cu") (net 2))
 (segment (start 221 69) (end 221 72) (width 0.6) (layer "F.Cu") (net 10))
 (segment (start 210 62.1) (end 210 69.124374) (width 0.6) (layer "F.Cu") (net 10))
 (segment (start 210 69.124374) (end 211.076626 70.201) (width 0.6) (layer "F.Cu") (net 10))
 (segment (start 221 72) (end 222 73) (width 0.6) (layer "F.Cu") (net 10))
 (segment (start 219.799 70.201) (end 221 69) (width 0.6) (layer "F.Cu") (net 10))
 (segment (start 211.076626 70.201) (end 219.799 70.201) (width 0.6) (layer "F.Cu") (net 10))
 (segment (start 209.2 61.3) (end 210 62.1) (width 0.6) (layer "F.Cu") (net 10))
 (segment (start 217 84) (end 224 91) (width 0.6) (layer "F.Cu") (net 15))
 (segment (start 216 84) (end 217 84) (width 0.6) (layer "F.Cu") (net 15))
 (segment (start 225.098001 87.098001) (end 225.098001 81.867) (width 0.6) (layer "F.Cu") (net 7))
 (segment (start 227.16 95) (end 227.16 91.36) (width 0.6) (layer "F.Cu") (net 7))
 (segment (start 226.8 91) (end 227 90.8) (width 0.6) (layer "F.Cu") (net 7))
 (segment (start 227.16 91.16) (end 227 91) (width 0.6) (layer "F.Cu") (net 7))
 (segment (start 227.16 91.36) (end 226.8 91) (width 0.6) (layer "F.Cu") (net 7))
 (segment (start 226.8 91) (end 226.8 88.8) (width 0.6) (layer "F.Cu") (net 7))
 (segment (start 226.600001 80.365) (end 227.4125 80.365) (width 0.6) (layer "F.Cu") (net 7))
 (segment (start 226.8 88.8) (end 225.098001 87.098001) (width 0.6) (layer "F.Cu") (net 7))
 (segment (start 225.098001 81.867) (end 226.600001 80.365) (width 0.6) (layer "F.Cu") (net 7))
 (segment (start 205 96) (end 205 91.2) (width 0.6) (layer "F.Cu") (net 14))
 (segment (start 205 91.2) (end 205.2 91) (width 0.6) (layer "F.Cu") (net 14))
 (segment (start 220.799 73.073206) (end 220.799 73.809424) (width 0.6) (layer "F.Cu") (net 1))
 (segment (start 223 74.010424) (end 223.290576 74.301) (width 0.6) (layer "F.Cu") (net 1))
 (segment (start 241.311 95.601024) (end 240.461024 96.451) (width 0.6) (layer "F.Cu") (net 1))
 (segment (start 225.901 73.901) (end 231 79) (width 0.6) (layer "F.Cu") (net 1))
 (segment (start 231 93.76) (end 232.24 95) (width 0.6) (layer "F.Cu") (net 1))
 (segment (start 231 79) (end 231 93.76) (width 0.6) (layer "F.Cu") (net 1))
 (segment (start 222.709424 74.301) (end 223 74.010424) (width 0.6) (layer "F.Cu") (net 1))
 (segment (start 211.65 73) (end 220.725794 73) (width 0.6) (layer "F.Cu") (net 1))
 (segment (start 223.290576 74.301) (end 224.709424 74.301) (width 0.6) (layer "F.Cu") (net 1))
 (segment (start 234.5875 81.635) (end 235.399999 81.635) (width 0.6) (layer "F.Cu") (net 1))
 (segment (start 233.691 96.451) (end 232.24 95) (width 0.6) (layer "F.Cu") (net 1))
 (segment (start 220.799 73.809424) (end 221.290576 74.301) (width 0.6) (layer "F.Cu") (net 1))
 (segment (start 240.461024 96.451) (end 233.691 96.451) (width 0.6) (layer "F.Cu") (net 1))
 (segment (start 241.311 87.546001) (end 241.311 95.601024) (width 0.6) (layer "F.Cu") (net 1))
 (segment (start 224.709424 74.301) (end 225.109424 73.901) (width 0.6) (layer "F.Cu") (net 1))
 (segment (start 235.399999 81.635) (end 241.311 87.546001) (width 0.6) (layer "F.Cu") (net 1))
 (segment (start 225.109424 73.901) (end 225.901 73.901) (width 0.6) (layer "F.Cu") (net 1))
 (segment (start 221.290576 74.301) (end 222.709424 74.301) (width 0.6) (layer "F.Cu") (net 1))
 (segment (start 220.725794 73) (end 220.799 73.073206) (width 0.6) (layer "F.Cu") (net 1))
 (segment (start 234.5875 82.905) (end 237.32 85.6375) (width 0.6) (layer "F.Cu") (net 3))
 (segment (start 237.32 85.6375) (end 237.32 95) (width 0.6) (layer "F.Cu") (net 3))
 (segment (start 237.32 95) (end 237 95) (width 0.6) (layer "F.Cu") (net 3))
 (segment (start 229.7 87.089254) (end 225.999 83.388254) (width 0.6) (layer "F.Cu") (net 8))
 (segment (start 226.785746 81.635) (end 227.4125 81.635) (width 0.6) (layer "F.Cu") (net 8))
 (segment (start 225.999 82.421746) (end 226.785746 81.635) (width 0.6) (layer "F.Cu") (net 8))
 (segment (start 229.7 95) (end 229.7 87.089254) (width 0.6) (layer "F.Cu") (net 8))
 (segment (start 225.999 83.388254) (end 225.999 82.421746) (width 0.6) (layer "F.Cu") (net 8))
 (segment (start 225.47 88.744206) (end 224.197001 87.471207) (width 0.6) (layer "F.Cu") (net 6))
 (segment (start 226.595795 79.095) (end 227.4125 79.095) (width 0.6) (layer "F.Cu") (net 6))
 (segment (start 224.62 95) (end 225 95) (width 0.6) (layer "F.Cu") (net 6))
 (segment (start 225.47 94.15) (end 225.47 88.744206) (width 0.6) (layer "F.Cu") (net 6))
 (segment (start 224.197001 87.471207) (end 224.197002 81.493793) (width 0.6) (layer "F.Cu") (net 6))
 (segment (start 224.62 95) (end 225.47 94.15) (width 0.6) (layer "F.Cu") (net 6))
 (segment (start 224.197002 81.493793) (end 226.595795 79.095) (width 0.6) (layer "F.Cu") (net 6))
 (segment (start 233.174 93.394) (end 234.78 95) (width 0.6) (layer "F.Cu") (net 4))
 (segment (start 227 73) (end 233.174 79.174) (width 0.6) (layer "F.Cu") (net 4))
 (segment (start 233.174 79.174) (end 233.174 79.578254) (width 0.6) (layer "F.Cu") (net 4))
 (segment (start 233.616746 80.021) (end 234.021 80.021) (width 0.6) (layer "F.Cu") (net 4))
 (segment (start 233.174 79.578254) (end 233.616746 80.021) (width 0.6) (layer "F.Cu") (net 4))
 (segment (start 234.021 80.021) (end 234.365 80.365) (width 0.6) (layer "F.Cu") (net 4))
 (segment (start 234.5875 80.365) (end 233.775001 80.365) (width 0.6) (layer "F.Cu") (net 4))
 (segment (start 234.365 80.365) (end 234.5875 80.365) (width 0.6) (layer "F.Cu") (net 4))
 (segment (start 233.775001 80.365) (end 233.174 80.966001) (width 0.6) (layer "F.Cu") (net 4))
 (segment (start 224 73) (end 227 73) (width 0.6) (layer "F.Cu") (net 4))
 (segment (start 233.174 80.966001) (end 233.174 93.394) (width 0.6) (layer "F.Cu") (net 4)))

